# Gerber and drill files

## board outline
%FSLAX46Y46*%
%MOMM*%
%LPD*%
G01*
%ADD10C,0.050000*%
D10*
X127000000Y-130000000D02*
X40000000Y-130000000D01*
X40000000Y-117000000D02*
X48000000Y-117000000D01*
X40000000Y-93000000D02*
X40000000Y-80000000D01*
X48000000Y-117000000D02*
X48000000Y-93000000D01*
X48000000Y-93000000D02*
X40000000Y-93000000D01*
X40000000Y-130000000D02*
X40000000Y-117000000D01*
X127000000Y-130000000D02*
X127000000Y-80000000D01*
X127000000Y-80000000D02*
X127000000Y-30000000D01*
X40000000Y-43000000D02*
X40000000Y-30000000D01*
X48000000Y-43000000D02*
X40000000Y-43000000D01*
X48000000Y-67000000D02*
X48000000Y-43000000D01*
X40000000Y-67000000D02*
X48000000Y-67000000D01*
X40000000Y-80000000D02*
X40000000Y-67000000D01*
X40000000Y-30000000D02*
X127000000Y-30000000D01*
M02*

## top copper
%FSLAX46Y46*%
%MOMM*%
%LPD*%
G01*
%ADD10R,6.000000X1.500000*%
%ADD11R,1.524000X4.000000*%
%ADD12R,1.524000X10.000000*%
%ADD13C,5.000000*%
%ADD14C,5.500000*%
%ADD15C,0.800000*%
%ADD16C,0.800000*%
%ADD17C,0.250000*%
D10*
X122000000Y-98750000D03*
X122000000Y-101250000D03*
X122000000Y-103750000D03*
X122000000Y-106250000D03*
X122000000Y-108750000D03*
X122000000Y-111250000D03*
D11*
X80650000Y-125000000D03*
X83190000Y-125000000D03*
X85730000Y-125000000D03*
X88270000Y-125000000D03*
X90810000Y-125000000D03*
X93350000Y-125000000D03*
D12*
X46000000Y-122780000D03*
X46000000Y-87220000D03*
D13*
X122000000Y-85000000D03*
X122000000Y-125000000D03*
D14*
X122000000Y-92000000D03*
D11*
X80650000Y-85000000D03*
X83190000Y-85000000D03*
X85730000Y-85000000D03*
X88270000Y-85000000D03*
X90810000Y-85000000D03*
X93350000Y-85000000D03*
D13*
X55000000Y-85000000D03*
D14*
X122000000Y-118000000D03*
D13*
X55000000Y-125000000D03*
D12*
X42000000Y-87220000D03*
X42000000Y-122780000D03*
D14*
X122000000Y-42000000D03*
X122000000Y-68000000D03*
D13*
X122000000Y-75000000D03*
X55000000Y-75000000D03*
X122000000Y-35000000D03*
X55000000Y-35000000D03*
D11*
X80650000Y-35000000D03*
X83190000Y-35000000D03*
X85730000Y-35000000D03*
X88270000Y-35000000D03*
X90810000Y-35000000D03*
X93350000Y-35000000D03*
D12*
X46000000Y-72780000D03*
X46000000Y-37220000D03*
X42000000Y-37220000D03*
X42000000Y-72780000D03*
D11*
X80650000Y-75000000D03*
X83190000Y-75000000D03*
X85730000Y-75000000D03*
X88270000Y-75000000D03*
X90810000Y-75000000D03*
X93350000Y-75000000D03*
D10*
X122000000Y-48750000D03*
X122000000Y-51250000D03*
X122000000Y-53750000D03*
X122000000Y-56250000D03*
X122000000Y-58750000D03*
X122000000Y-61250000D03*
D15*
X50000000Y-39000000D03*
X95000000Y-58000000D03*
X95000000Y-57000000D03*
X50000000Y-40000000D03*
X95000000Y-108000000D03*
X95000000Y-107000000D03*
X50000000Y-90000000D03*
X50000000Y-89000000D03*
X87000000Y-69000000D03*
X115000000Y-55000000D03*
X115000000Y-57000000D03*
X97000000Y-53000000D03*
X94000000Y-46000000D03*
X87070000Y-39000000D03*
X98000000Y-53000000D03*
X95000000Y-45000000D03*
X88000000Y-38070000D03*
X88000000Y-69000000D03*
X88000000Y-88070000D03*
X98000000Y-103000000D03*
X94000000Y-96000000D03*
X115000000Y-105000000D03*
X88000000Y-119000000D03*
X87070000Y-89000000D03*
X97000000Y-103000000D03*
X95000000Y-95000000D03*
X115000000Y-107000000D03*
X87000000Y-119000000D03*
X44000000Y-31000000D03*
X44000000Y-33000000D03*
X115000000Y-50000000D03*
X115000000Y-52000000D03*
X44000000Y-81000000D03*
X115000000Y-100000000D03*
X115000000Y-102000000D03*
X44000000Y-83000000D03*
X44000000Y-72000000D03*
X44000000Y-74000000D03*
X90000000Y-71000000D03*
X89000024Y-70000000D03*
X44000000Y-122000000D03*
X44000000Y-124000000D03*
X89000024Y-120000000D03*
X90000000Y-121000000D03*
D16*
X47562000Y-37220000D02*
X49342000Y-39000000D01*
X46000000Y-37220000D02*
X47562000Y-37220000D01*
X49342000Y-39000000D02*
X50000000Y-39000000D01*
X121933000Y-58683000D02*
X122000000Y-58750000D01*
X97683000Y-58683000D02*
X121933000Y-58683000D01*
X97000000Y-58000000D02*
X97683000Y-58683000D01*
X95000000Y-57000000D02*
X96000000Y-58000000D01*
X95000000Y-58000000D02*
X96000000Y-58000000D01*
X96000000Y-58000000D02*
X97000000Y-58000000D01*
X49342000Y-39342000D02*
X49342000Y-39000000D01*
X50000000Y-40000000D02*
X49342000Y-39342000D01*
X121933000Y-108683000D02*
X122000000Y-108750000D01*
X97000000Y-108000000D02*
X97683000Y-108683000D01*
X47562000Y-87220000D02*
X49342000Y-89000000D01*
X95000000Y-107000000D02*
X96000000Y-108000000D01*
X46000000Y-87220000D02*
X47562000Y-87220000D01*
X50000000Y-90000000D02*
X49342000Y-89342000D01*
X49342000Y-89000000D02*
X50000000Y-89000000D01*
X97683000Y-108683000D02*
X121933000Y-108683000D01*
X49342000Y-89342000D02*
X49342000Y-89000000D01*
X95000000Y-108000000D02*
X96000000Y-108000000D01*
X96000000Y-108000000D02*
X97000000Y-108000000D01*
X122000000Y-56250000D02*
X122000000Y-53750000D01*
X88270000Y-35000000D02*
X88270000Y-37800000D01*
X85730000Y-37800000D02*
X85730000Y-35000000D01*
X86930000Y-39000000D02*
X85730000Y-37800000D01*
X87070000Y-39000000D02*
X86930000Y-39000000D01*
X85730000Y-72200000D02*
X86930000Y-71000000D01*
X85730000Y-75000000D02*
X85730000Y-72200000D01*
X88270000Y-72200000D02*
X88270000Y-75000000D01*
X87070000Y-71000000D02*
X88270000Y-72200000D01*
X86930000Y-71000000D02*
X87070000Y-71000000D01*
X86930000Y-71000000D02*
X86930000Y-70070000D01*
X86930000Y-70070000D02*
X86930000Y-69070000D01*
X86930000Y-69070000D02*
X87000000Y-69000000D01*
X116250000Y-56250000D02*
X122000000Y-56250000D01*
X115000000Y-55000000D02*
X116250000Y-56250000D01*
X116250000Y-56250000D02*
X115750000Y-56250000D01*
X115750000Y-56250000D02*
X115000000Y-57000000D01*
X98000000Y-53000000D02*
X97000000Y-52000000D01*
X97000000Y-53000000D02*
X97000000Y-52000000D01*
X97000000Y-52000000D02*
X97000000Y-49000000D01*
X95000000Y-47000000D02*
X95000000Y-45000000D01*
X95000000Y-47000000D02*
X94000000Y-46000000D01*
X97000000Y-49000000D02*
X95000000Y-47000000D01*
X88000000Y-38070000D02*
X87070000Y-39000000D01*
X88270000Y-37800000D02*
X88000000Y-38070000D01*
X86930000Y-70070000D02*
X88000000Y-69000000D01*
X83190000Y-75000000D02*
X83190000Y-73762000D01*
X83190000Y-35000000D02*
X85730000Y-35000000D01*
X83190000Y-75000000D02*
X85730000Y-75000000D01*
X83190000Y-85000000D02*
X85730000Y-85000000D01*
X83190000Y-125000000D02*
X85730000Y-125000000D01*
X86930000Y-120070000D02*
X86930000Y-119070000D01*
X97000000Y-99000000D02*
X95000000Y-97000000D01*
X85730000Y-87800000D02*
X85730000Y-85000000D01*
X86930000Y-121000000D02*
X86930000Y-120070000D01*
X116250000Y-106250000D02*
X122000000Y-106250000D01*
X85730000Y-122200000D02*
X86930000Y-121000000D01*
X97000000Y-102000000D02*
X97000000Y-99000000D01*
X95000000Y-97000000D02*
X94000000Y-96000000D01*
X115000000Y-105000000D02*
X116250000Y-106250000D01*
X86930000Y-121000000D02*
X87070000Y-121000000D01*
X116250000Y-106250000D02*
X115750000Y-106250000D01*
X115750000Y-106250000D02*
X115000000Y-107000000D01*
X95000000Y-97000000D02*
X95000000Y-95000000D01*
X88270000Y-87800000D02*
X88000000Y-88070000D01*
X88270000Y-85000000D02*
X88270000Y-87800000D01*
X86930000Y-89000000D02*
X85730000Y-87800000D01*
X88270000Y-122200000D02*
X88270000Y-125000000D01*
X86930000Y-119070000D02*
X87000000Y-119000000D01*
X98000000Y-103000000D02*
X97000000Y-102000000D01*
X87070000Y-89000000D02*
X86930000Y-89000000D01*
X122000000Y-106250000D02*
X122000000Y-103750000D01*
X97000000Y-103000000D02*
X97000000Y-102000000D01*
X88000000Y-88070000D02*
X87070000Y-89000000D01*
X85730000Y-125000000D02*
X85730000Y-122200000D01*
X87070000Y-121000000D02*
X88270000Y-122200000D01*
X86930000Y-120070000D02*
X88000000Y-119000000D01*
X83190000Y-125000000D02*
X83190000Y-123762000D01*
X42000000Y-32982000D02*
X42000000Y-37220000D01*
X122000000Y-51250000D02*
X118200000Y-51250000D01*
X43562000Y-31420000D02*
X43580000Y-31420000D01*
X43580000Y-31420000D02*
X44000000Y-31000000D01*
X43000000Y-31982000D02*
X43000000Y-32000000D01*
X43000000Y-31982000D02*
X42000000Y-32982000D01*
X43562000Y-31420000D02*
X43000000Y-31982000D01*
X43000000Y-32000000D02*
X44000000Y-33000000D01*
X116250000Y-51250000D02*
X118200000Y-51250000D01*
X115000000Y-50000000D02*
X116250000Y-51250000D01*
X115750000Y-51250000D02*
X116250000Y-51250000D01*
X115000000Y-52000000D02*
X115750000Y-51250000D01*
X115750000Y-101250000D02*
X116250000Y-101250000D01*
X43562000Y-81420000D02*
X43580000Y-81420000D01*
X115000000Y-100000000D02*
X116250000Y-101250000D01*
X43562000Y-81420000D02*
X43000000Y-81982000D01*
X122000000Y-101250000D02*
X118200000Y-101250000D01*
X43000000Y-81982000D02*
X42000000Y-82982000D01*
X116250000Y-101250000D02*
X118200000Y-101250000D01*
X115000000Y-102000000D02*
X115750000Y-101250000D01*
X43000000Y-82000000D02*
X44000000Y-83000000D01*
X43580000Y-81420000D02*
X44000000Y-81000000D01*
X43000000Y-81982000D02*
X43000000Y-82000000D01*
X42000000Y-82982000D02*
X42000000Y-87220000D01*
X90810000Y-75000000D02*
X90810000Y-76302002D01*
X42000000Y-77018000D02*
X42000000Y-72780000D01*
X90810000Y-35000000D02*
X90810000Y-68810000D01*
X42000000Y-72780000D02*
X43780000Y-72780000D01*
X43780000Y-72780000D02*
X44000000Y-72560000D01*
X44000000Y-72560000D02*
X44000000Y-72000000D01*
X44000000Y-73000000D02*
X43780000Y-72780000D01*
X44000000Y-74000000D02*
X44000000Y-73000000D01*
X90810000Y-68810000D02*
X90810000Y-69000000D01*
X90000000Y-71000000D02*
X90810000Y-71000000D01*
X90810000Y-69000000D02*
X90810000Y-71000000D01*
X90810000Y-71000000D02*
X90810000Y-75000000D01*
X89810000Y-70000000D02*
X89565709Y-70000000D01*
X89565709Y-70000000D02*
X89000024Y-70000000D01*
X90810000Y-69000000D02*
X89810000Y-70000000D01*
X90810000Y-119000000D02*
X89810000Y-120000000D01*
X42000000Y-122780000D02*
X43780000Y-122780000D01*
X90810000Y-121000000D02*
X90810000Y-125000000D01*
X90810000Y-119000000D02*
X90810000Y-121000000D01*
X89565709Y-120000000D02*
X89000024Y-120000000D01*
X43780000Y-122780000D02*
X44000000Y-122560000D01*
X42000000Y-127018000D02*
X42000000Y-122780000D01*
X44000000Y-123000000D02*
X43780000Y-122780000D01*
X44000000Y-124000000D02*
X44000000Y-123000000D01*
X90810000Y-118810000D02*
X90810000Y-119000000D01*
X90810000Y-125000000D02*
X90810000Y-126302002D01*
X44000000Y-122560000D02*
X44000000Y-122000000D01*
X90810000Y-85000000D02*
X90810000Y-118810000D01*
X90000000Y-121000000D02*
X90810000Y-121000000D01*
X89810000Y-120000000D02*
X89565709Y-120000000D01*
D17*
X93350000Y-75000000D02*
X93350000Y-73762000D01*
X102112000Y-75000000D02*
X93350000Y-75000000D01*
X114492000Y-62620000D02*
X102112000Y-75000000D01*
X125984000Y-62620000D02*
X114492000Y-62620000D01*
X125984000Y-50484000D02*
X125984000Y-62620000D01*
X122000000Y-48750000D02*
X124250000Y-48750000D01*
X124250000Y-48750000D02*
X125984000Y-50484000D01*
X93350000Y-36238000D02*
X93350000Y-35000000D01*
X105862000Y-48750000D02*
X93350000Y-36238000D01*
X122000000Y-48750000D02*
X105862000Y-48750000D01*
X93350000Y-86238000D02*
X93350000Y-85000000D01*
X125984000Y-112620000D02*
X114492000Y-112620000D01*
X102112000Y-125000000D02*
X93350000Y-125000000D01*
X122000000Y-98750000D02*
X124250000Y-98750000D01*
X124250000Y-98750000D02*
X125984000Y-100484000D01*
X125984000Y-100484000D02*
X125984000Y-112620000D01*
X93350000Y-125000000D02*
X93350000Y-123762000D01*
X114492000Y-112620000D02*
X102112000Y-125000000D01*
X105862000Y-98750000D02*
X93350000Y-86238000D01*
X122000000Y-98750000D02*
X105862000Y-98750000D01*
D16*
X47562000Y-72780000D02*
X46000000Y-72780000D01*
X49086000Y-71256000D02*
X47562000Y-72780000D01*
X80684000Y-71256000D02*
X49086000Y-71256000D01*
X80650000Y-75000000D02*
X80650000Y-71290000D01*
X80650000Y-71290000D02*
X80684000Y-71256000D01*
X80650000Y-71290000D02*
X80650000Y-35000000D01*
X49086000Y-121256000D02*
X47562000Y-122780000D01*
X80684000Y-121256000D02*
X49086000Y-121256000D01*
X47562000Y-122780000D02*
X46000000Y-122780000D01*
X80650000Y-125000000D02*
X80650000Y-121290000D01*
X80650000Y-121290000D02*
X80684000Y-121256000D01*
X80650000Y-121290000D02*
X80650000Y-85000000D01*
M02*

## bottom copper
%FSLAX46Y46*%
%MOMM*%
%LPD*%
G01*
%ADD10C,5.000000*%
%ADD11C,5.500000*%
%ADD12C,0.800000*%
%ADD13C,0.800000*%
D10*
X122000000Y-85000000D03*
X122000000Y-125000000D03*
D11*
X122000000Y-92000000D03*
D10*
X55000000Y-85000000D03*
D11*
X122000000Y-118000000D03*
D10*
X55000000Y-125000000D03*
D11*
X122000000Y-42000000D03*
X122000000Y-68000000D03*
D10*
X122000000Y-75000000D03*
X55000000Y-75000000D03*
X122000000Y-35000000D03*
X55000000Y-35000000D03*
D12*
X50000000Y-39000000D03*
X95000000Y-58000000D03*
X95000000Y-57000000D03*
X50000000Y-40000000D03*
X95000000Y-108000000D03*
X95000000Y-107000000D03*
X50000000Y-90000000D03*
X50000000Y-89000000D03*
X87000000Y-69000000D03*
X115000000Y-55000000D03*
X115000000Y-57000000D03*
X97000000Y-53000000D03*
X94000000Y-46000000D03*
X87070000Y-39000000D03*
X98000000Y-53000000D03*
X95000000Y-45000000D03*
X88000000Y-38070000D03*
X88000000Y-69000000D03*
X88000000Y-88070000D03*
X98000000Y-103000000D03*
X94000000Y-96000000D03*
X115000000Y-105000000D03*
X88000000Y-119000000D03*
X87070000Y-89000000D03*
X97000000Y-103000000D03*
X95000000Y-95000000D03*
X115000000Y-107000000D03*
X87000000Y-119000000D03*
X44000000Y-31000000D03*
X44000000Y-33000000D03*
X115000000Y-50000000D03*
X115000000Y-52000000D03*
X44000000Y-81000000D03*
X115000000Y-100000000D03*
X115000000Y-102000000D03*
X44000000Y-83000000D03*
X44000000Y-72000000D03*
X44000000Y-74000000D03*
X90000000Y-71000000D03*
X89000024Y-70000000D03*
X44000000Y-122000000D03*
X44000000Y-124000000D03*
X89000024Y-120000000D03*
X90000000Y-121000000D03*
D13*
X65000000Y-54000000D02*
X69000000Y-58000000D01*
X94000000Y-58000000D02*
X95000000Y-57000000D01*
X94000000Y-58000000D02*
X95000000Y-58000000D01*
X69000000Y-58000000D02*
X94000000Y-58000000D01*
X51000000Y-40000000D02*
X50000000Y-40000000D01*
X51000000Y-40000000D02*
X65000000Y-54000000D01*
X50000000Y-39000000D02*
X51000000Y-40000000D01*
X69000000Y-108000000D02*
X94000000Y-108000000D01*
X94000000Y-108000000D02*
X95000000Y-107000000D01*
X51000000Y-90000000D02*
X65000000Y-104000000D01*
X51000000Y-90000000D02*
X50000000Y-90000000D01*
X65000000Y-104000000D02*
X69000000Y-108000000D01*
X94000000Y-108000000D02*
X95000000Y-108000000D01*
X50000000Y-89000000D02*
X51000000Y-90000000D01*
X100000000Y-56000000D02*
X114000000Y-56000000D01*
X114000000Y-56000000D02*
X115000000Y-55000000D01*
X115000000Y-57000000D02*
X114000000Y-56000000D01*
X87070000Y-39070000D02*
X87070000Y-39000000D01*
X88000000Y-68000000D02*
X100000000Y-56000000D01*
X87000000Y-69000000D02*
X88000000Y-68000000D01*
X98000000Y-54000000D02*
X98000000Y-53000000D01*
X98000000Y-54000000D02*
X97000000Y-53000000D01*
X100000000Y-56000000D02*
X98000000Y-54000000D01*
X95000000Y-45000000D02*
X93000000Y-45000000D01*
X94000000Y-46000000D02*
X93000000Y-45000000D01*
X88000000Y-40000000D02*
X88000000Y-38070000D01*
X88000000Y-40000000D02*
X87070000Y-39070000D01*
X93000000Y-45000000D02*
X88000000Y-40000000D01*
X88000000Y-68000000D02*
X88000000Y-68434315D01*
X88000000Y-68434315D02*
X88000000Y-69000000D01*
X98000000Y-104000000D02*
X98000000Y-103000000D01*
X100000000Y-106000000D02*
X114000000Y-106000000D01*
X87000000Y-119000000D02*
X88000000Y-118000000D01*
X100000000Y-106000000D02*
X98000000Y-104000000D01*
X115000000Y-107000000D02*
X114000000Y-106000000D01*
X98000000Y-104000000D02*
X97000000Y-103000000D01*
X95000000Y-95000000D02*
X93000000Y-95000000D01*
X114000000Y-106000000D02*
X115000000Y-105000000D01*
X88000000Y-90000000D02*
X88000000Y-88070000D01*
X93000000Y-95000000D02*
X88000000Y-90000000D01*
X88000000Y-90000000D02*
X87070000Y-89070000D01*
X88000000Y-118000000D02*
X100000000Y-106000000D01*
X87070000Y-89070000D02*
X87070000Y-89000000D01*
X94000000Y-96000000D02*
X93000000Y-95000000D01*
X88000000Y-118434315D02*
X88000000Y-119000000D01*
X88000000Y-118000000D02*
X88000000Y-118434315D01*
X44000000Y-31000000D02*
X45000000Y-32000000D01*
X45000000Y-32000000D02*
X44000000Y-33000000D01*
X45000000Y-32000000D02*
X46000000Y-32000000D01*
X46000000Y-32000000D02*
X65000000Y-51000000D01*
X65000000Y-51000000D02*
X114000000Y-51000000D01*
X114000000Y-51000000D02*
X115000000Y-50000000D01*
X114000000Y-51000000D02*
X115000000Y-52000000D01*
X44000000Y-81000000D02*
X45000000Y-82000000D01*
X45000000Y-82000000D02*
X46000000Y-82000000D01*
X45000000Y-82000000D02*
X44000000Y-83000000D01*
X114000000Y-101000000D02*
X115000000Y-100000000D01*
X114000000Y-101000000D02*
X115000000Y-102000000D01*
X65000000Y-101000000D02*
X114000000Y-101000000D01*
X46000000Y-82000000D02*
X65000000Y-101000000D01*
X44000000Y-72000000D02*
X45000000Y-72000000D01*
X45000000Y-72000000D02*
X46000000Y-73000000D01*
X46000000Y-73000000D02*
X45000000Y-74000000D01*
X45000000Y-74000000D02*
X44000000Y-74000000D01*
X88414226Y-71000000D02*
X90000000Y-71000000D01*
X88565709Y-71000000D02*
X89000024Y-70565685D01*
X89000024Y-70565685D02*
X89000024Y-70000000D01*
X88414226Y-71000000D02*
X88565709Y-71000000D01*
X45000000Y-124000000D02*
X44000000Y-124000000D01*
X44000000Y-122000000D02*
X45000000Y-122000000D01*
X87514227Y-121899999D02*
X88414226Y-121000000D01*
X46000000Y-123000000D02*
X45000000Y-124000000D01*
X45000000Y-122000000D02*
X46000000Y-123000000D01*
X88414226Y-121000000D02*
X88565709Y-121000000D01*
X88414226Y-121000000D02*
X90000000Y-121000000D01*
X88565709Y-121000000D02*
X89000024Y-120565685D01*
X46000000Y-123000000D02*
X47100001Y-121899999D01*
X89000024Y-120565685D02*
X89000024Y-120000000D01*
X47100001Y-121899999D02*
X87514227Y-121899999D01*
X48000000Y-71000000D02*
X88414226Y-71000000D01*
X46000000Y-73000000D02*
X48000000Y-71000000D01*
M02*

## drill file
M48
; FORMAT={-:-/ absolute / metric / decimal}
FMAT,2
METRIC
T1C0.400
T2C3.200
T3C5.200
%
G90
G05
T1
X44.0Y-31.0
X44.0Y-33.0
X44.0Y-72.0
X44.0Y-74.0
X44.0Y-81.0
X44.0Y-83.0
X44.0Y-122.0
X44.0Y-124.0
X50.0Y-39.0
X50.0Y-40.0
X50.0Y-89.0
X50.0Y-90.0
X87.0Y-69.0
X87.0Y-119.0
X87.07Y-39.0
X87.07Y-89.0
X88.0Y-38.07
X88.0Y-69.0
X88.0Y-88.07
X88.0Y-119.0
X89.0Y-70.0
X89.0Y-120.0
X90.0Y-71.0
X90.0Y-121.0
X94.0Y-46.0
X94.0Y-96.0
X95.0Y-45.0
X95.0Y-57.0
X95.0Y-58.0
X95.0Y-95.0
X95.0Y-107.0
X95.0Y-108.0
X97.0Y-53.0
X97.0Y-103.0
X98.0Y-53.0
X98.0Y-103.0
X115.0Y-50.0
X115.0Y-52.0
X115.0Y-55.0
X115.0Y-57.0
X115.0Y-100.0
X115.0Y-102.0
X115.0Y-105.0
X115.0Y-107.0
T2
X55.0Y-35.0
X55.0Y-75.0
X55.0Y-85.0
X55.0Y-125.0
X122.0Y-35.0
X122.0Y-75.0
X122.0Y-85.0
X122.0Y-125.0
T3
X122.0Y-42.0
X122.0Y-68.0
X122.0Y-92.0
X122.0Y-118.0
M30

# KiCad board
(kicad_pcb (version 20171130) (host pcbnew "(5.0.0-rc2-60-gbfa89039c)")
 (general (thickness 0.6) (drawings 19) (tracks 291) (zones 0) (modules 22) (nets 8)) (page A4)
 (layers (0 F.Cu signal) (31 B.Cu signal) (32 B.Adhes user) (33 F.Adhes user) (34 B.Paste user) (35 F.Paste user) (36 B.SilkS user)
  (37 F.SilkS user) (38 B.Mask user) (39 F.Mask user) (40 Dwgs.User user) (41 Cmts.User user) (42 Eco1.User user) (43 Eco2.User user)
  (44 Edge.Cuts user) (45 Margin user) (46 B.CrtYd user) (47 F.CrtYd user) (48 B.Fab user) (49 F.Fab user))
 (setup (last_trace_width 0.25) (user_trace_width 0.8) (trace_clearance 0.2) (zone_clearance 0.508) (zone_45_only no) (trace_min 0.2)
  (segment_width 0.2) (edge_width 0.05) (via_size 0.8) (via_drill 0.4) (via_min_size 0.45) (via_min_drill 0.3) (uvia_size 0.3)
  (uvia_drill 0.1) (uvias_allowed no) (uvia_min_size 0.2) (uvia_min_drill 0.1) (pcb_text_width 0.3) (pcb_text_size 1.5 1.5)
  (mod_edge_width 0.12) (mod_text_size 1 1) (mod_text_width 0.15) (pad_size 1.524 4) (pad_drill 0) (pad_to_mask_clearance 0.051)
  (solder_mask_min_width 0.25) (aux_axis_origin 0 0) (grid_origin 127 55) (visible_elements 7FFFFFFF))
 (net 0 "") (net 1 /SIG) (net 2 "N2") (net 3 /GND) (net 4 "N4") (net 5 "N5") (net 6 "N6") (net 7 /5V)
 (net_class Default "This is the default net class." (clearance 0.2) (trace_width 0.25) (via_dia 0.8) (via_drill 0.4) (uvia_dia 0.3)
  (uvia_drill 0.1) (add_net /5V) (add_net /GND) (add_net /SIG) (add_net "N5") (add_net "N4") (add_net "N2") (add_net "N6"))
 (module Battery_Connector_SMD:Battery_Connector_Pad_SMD (layer F.Cu) (at 122 105 90)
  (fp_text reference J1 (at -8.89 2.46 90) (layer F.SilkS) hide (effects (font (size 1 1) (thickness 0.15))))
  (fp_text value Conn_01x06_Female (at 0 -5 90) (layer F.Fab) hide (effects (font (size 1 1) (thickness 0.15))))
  (pad 6 smd rect (at 6.25 0 90) (size 1.5 6) (layers F.Cu F.Mask) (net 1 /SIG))
  (pad 5 smd rect (at 3.75 0 90) (size 1.5 6) (layers F.Cu F.Mask) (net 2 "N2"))
  (pad 4 smd rect (at 1.25 0 90) (size 1.5 6) (layers F.Cu F.Mask) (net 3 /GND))
  (pad 3 smd rect (at -1.25 0 90) (size 1.5 6) (layers F.Cu F.Mask) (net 3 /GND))
  (pad 2 smd rect (at -3.75 0 90) (size 1.5 6) (layers F.Cu F.Mask) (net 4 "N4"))
  (pad 1 smd rect (at -6.25 0 90) (size 1.5 6) (layers F.Cu F.Mask) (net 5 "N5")))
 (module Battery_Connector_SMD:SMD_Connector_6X (layer F.Cu) (at 87 125 180)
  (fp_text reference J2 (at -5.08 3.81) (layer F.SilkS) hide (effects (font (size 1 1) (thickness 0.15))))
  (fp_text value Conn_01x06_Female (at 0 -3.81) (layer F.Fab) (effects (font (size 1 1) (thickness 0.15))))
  (pad 6 smd rect (at 6.35 0 180) (size 1.524 4) (layers F.Cu F.Paste F.Mask) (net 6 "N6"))
  (pad 5 smd rect (at 3.81 0 180) (size 1.524 4) (layers F.Cu F.Paste F.Mask) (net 3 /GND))
  (pad 4 smd rect (at 1.27 0 180) (size 1.524 4) (layers F.Cu F.Paste F.Mask) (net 3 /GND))
  (pad 3 smd rect (at -1.27 0 180) (size 1.524 4) (layers F.Cu F.Paste F.Mask) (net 3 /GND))
  (pad 2 smd rect (at -3.81 0 180) (size 1.524 4) (layers F.Cu F.Paste F.Mask) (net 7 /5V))
  (pad 1 smd rect (at -6.35 0 180) (size 1.524 4) (layers F.Cu F.Paste F.Mask) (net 1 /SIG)))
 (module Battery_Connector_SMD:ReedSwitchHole (layer F.Cu) (at 46 105)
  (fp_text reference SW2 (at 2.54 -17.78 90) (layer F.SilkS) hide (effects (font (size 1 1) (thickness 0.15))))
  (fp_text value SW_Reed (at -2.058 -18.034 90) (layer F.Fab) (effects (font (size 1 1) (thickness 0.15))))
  (pad 2 smd rect (at 0 17.78) (size 1.524 10) (layers F.Cu F.Mask) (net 6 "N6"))
  (pad 1 smd rect (at 0 -17.78) (size 1.524 10) (layers F.Cu F.Mask) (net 4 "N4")))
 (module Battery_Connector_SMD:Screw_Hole (layer F.Cu) (at 122 85)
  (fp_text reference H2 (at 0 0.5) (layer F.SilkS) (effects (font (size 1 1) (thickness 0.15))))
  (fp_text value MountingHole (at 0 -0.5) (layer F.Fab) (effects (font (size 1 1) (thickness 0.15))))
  (pad 1 thru_hole circle (at 0 0) (size 5 5) (drill 3.2) (layers *.Cu *.Mask)))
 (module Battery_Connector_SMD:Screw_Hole (layer F.Cu) (at 122 125)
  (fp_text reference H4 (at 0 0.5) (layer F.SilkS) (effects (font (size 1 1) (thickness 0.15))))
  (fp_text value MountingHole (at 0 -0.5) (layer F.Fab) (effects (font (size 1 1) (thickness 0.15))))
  (pad 1 thru_hole circle (at 0 0) (size 5 5) (drill 3.2) (layers *.Cu *.Mask)))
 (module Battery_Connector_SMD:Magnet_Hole (layer F.Cu) (at 122 92)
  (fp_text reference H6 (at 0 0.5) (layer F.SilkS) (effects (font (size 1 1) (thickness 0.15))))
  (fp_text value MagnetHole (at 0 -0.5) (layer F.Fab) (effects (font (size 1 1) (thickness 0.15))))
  (pad 1 thru_hole circle (at 0 0) (size 5.5 5.5) (drill 5.2) (layers *.Cu *.Mask)))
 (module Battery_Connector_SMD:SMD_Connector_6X (layer F.Cu) (at 87 85 180)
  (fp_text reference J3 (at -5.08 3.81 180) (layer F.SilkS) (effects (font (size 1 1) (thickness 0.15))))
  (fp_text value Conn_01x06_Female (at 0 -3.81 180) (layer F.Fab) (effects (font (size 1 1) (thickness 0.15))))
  (pad 6 smd rect (at 6.35 0 180) (size 1.524 4) (layers F.Cu F.Paste F.Mask) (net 6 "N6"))
  (pad 5 smd rect (at 3.81 0 180) (size 1.524 4) (layers F.Cu F.Paste F.Mask) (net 3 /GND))
  (pad 4 smd rect (at 1.27 0 180) (size 1.524 4) (layers F.Cu F.Paste F.Mask) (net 3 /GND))
  (pad 3 smd rect (at -1.27 0 180) (size 1.524 4) (layers F.Cu F.Paste F.Mask) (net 3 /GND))
  (pad 2 smd rect (at -3.81 0 180) (size 1.524 4) (layers F.Cu F.Paste F.Mask) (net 7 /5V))
  (pad 1 smd rect (at -6.35 0 180) (size 1.524 4) (layers F.Cu F.Paste F.Mask) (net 1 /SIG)))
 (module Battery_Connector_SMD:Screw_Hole (layer F.Cu) (at 55 85)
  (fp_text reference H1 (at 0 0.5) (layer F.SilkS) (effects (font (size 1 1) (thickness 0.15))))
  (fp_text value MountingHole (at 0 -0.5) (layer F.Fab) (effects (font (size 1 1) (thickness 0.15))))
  (pad 1 thru_hole circle (at 0 0) (size 5 5) (drill 3.2) (layers *.Cu *.Mask)))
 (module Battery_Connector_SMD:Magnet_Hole (layer F.Cu) (at 122 118)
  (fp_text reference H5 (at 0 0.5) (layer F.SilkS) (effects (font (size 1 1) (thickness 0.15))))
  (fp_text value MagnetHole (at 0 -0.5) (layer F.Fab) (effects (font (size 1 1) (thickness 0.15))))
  (pad 1 thru_hole circle (at 0 0) (size 5.5 5.5) (drill 5.2) (layers *.Cu *.Mask)))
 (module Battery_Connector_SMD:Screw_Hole (layer F.Cu) (at 55 125)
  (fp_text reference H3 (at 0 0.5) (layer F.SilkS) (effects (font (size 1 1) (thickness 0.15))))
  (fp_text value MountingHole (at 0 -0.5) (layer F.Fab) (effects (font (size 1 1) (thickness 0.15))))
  (pad 1 thru_hole circle (at 0 0) (size 5 5) (drill 3.2) (layers *.Cu *.Mask)))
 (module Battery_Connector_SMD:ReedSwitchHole (layer F.Cu) (at 42 105 180)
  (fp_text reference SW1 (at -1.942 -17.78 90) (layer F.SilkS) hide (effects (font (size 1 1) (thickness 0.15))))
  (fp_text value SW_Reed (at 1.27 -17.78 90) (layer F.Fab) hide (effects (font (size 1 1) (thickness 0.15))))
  (pad 2 smd rect (at 0 17.78 180) (size 1.524 10) (layers F.Cu F.Mask) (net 2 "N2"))
  (pad 1 smd rect (at 0 -17.78 180) (size 1.524 10) (layers F.Cu F.Mask) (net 7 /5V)))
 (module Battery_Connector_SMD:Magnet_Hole (layer F.Cu) (at 122 42)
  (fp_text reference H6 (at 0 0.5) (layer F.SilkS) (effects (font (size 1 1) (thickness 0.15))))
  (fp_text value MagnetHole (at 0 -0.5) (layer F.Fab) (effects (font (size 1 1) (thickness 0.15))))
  (pad 1 thru_hole circle (at 0 0) (size 5.5 5.5) (drill 5.2) (layers *.Cu *.Mask)))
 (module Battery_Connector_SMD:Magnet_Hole (layer F.Cu) (at 122 68)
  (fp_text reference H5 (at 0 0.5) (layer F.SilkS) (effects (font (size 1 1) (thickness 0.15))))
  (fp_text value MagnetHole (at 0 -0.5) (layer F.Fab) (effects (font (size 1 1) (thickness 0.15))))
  (pad 1 thru_hole circle (at 0 0) (size 5.5 5.5) (drill 5.2) (layers *.Cu *.Mask)))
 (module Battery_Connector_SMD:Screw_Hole (layer F.Cu) (at 122 75)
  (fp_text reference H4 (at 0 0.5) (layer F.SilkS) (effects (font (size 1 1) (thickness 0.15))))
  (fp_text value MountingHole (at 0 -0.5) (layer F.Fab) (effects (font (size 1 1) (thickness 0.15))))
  (pad 1 thru_hole circle (at 0 0) (size 5 5) (drill 3.2) (layers *.Cu *.Mask)))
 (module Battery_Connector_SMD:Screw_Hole (layer F.Cu) (at 55 75)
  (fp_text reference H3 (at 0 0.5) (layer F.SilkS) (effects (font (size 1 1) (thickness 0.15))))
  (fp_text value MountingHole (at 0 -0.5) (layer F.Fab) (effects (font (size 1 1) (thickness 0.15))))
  (pad 1 thru_hole circle (at 0 0) (size 5 5) (drill 3.2) (layers *.Cu *.Mask)))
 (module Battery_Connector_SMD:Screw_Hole (layer F.Cu) (at 122 35)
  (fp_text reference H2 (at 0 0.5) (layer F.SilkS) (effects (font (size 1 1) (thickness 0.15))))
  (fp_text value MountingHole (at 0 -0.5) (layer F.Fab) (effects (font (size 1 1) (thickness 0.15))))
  (pad 1 thru_hole circle (at 0 0) (size 5 5) (drill 3.2) (layers *.Cu *.Mask)))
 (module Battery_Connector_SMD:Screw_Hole (layer F.Cu) (at 55 35)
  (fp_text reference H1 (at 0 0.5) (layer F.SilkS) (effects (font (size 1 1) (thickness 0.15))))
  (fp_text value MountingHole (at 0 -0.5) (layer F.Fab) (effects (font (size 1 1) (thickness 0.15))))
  (pad 1 thru_hole circle (at 0 0) (size 5 5) (drill 3.2) (layers *.Cu *.Mask)))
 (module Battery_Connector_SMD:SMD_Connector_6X (layer F.Cu) (at 87 35 180)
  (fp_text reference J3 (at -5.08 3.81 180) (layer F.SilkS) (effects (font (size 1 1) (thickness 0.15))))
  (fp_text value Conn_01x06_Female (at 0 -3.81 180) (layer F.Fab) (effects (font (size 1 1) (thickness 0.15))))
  (pad 6 smd rect (at 6.35 0 180) (size 1.524 4) (layers F.Cu F.Paste F.Mask) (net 6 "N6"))
  (pad 5 smd rect (at 3.81 0 180) (size 1.524 4) (layers F.Cu F.Paste F.Mask) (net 3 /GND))
  (pad 4 smd rect (at 1.27 0 180) (size 1.524 4) (layers F.Cu F.Paste F.Mask) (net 3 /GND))
  (pad 3 smd rect (at -1.27 0 180) (size 1.524 4) (layers F.Cu F.Paste F.Mask) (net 3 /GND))
  (pad 2 smd rect (at -3.81 0 180) (size 1.524 4) (layers F.Cu F.Paste F.Mask) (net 7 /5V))
  (pad 1 smd rect (at -6.35 0 180) (size 1.524 4) (layers F.Cu F.Paste F.Mask) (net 1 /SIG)))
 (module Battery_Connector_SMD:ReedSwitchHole (layer F.Cu) (at 46 55)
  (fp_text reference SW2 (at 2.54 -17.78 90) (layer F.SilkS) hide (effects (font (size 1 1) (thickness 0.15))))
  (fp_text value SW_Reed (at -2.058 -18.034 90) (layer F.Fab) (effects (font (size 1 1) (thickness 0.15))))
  (pad 2 smd rect (at 0 17.78) (size 1.524 10) (layers F.Cu F.Mask) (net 6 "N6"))
  (pad 1 smd rect (at 0 -17.78) (size 1.524 10) (layers F.Cu F.Mask) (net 4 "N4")))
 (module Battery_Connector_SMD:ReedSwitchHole (layer F.Cu) (at 42 55 180)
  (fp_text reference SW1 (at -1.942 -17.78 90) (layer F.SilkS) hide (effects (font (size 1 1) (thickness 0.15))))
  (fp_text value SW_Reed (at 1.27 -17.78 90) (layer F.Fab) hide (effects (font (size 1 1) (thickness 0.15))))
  (pad 2 smd rect (at 0 17.78 180) (size 1.524 10) (layers F.Cu F.Mask) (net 2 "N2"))
  (pad 1 smd rect (at 0 -17.78 180) (size 1.524 10) (layers F.Cu F.Mask) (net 7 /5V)))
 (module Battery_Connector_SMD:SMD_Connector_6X (layer F.Cu) (at 87 75 180)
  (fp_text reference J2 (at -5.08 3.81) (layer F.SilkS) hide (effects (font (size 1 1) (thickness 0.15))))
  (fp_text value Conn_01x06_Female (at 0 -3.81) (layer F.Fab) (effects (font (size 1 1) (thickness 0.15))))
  (pad 6 smd rect (at 6.35 0 180) (size 1.524 4) (layers F.Cu F.Paste F.Mask) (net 6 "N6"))
  (pad 5 smd rect (at 3.81 0 180) (size 1.524 4) (layers F.Cu F.Paste F.Mask) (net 3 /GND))
  (pad 4 smd rect (at 1.27 0 180) (size 1.524 4) (layers F.Cu F.Paste F.Mask) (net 3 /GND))
  (pad 3 smd rect (at -1.27 0 180) (size 1.524 4) (layers F.Cu F.Paste F.Mask) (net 3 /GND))
  (pad 2 smd rect (at -3.81 0 180) (size 1.524 4) (layers F.Cu F.Paste F.Mask) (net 7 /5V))
  (pad 1 smd rect (at -6.35 0 180) (size 1.524 4) (layers F.Cu F.Paste F.Mask) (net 1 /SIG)))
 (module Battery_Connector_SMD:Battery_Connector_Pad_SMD (layer F.Cu) (at 122 55 90)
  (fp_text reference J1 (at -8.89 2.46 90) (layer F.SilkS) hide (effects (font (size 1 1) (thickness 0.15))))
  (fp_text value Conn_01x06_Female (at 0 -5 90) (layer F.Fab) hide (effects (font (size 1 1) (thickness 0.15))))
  (pad 6 smd rect (at 6.25 0 90) (size 1.5 6) (layers F.Cu F.Mask) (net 1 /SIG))
  (pad 5 smd rect (at 3.75 0 90) (size 1.5 6) (layers F.Cu F.Mask) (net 2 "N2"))
  (pad 4 smd rect (at 1.25 0 90) (size 1.5 6) (layers F.Cu F.Mask) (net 3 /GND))
  (pad 3 smd rect (at -1.25 0 90) (size 1.5 6) (layers F.Cu F.Mask) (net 3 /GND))
  (pad 2 smd rect (at -3.75 0 90) (size 1.5 6) (layers F.Cu F.Mask) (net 4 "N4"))
  (pad 1 smd rect (at -6.25 0 90) (size 1.5 6) (layers F.Cu F.Mask) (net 5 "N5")))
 (gr_line (start 127 130) (end 40 130) (layer Edge.Cuts) (width 0.05))
 (gr_line (start 40 117) (end 48 117) (layer Edge.Cuts) (width 0.05))
 (gr_line (start 40 93) (end 40 80) (layer Edge.Cuts) (width 0.05))
 (gr_line (start 48 117) (end 48 93) (layer Edge.Cuts) (width 0.05))
 (gr_line (start 48 93) (end 40 93) (layer Edge.Cuts) (width 0.05))
 (gr_line (start 40 130) (end 40 117) (layer Edge.Cuts) (width 0.05))
 (gr_line (start 127 130) (end 127 80) (layer Edge.Cuts) (width 0.05))
 (gr_line (start 127 80) (end 127 30) (layer Edge.Cuts) (width 0.05))
 (gr_line (start 40 43) (end 40 30) (layer Edge.Cuts) (width 0.05))
 (gr_line (start 48 43) (end 40 43) (layer Edge.Cuts) (width 0.05))
 (gr_line (start 48 67) (end 48 43) (layer Edge.Cuts) (width 0.05))
 (gr_line (start 40 67) (end 48 67) (layer Edge.Cuts) (width 0.05))
 (gr_line (start 40 80) (end 40 67) (layer Edge.Cuts) (width 0.05))
 (gr_line (start 40 30) (end 127 30) (layer Edge.Cuts) (width 0.05))
 (segment (start 47.562 37.22) (end 49.342 39) (width 0.8) (layer F.Cu) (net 4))
 (segment (start 46 37.22) (end 47.562 37.22) (width 0.8) (layer F.Cu) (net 4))
 (via (at 50 39) (size 0.8) (drill 0.4) (layers F.Cu B.Cu) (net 4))
 (segment (start 49.342 39) (end 50 39) (width 0.8) (layer F.Cu) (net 4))
 (segment (start 65 54) (end 69 58) (width 0.8) (layer B.Cu) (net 4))
 (via (at 95 58) (size 0.8) (drill 0.4) (layers F.Cu B.Cu) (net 4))
 (segment (start 121.933 58.683) (end 122 58.75) (width 0.8) (layer F.Cu) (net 4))
 (segment (start 97.683 58.683) (end 121.933 58.683) (width 0.8) (layer F.Cu) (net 4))
 (segment (start 97 58) (end 97.683 58.683) (width 0.8) (layer F.Cu) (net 4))
 (via (at 95 57) (size 0.8) (drill 0.4) (layers F.Cu B.Cu) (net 4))
 (segment (start 94 58) (end 95 57) (width 0.8) (layer B.Cu) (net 4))
 (segment (start 94 58) (end 95 58) (width 0.8) (layer B.Cu) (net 4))
 (segment (start 69 58) (end 94 58) (width 0.8) (layer B.Cu) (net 4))
 (segment (start 95 57) (end 96 58) (width 0.8) (layer F.Cu) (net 4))
 (segment (start 95 58) (end 96 58) (width 0.8) (layer F.Cu) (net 4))
 (segment (start 96 58) (end 97 58) (width 0.8) (layer F.Cu) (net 4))
 (via (at 50 40) (size 0.8) (drill 0.4) (layers F.Cu B.Cu) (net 4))
 (segment (start 51 40) (end 50 40) (width 0.8) (layer B.Cu) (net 4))
 (segment (start 51 40) (end 65 54) (width 0.8) (layer B.Cu) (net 4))
 (segment (start 50 39) (end 51 40) (width 0.8) (layer B.Cu) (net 4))
 (segment (start 49.342 39.342) (end 49.342 39) (width 0.8) (layer F.Cu) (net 4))
 (segment (start 50 40) (end 49.342 39.342) (width 0.8) (layer F.Cu) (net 4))
 (segment (start 121.933 108.683) (end 122 108.75) (width 0.8) (layer F.Cu) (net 4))
 (segment (start 69 108) (end 94 108) (width 0.8) (layer B.Cu) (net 4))
 (segment (start 94 108) (end 95 107) (width 0.8) (layer B.Cu) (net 4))
 (segment (start 51 90) (end 65 104) (width 0.8) (layer B.Cu) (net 4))
 (segment (start 97 108) (end 97.683 108.683) (width 0.8) (layer F.Cu) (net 4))
 (segment (start 47.562 87.22) (end 49.342 89) (width 0.8) (layer F.Cu) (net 4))
 (segment (start 95 107) (end 96 108) (width 0.8) (layer F.Cu) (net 4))
 (segment (start 51 90) (end 50 90) (width 0.8) (layer B.Cu) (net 4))
 (segment (start 46 87.22) (end 47.562 87.22) (width 0.8) (layer F.Cu) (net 4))
 (segment (start 50 90) (end 49.342 89.342) (width 0.8) (layer F.Cu) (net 4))
 (segment (start 49.342 89) (end 50 89) (width 0.8) (layer F.Cu) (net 4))
 (segment (start 65 104) (end 69 108) (width 0.8) (layer B.Cu) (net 4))
 (segment (start 94 108) (end 95 108) (width 0.8) (layer B.Cu) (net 4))
 (segment (start 97.683 108.683) (end 121.933 108.683) (width 0.8) (layer F.Cu) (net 4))
 (segment (start 49.342 89.342) (end 49.342 89) (width 0.8) (layer F.Cu) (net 4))
 (segment (start 95 108) (end 96 108) (width 0.8) (layer F.Cu) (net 4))
 (segment (start 96 108) (end 97 108) (width 0.8) (layer F.Cu) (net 4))
 (segment (start 50 89) (end 51 90) (width 0.8) (layer B.Cu) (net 4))
 (via (at 95 108) (size 0.8) (drill 0.4) (layers F.Cu B.Cu) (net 4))
 (via (at 95 107) (size 0.8) (drill 0.4) (layers F.Cu B.Cu) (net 4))
 (via (at 50 90) (size 0.8) (drill 0.4) (layers F.Cu B.Cu) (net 4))
 (via (at 50 89) (size 0.8) (drill 0.4) (layers F.Cu B.Cu) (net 4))
 (segment (start 122 56.25) (end 122 53.75) (width 0.8) (layer F.Cu) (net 3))
 (segment (start 88.27 35) (end 88.27 37.8) (width 0.8) (layer F.Cu) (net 3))
 (segment (start 85.73 37.8) (end 85.73 35) (width 0.8) (layer F.Cu) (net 3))
 (segment (start 86.93 39) (end 85.73 37.8) (width 0.8) (layer F.Cu) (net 3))
 (segment (start 87.07 39) (end 86.93 39) (width 0.8) (layer F.Cu) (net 3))
 (segment (start 85.73 72.2) (end 86.93 71) (width 0.8) (layer F.Cu) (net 3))
 (segment (start 85.73 75) (end 85.73 72.2) (width 0.8) (layer F.Cu) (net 3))
 (segment (start 88.27 72.2) (end 88.27 75) (width 0.8) (layer F.Cu) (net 3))
 (segment (start 87.07 71) (end 88.27 72.2) (width 0.8) (layer F.Cu) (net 3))
 (segment (start 86.93 71) (end 87.07 71) (width 0.8) (layer F.Cu) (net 3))
 (segment (start 86.93 71) (end 86.93 70.07) (width 0.8) (layer F.Cu) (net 3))
 (via (at 87 69) (size 0.8) (drill 0.4) (layers F.Cu B.Cu) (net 3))
 (segment (start 86.93 70.07) (end 86.93 69.07) (width 0.8) (layer F.Cu) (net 3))
 (segment (start 86.93 69.07) (end 87 69) (width 0.8) (layer F.Cu) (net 3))
 (segment (start 100 56) (end 114 56) (width 0.8) (layer B.Cu) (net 3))
 (via (at 115 55) (size 0.8) (drill 0.4) (layers F.Cu B.Cu) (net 3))
 (segment (start 114 56) (end 115 55) (width 0.8) (layer B.Cu) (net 3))
 (segment (start 116.25 56.25) (end 122 56.25) (width 0.8) (layer F.Cu) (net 3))
 (segment (start 115 55) (end 116.25 56.25) (width 0.8) (layer F.Cu) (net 3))
 (via (at 115 57) (size 0.8) (drill 0.4) (layers F.Cu B.Cu) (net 3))
 (segment (start 116.25 56.25) (end 115.75 56.25) (width 0.8) (layer F.Cu) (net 3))
 (segment (start 115.75 56.25) (end 115 57) (width 0.8) (layer F.Cu) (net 3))
 (segment (start 115 57) (end 114 56) (width 0.8) (layer B.Cu) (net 3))
 (via (at 97 53) (size 0.8) (drill 0.4) (layers F.Cu B.Cu) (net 3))
 (via (at 94 46) (size 0.8) (drill 0.4) (layers F.Cu B.Cu) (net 3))
 (via (at 87.07 39) (size 0.8) (drill 0.4) (layers F.Cu B.Cu) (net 3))
 (segment (start 87.07 39.07) (end 87.07 39) (width 0.8) (layer B.Cu) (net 3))
 (segment (start 88 68) (end 100 56) (width 0.8) (layer B.Cu) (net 3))
 (segment (start 87 69) (end 88 68) (width 0.8) (layer B.Cu) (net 3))
 (via (at 98 53) (size 0.8) (drill 0.4) (layers F.Cu B.Cu) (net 3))
 (segment (start 98 54) (end 98 53) (width 0.8) (layer B.Cu) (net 3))
 (segment (start 98 54) (end 97 53) (width 0.8) (layer B.Cu) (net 3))
 (segment (start 100 56) (end 98 54) (width 0.8) (layer B.Cu) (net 3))
 (segment (start 98 53) (end 97 52) (width 0.8) (layer F.Cu) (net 3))
 (segment (start 97 53) (end 97 52) (width 0.8) (layer F.Cu) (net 3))
 (segment (start 97 52) (end 97 49) (width 0.8) (layer F.Cu) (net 3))
 (via (at 95 45) (size 0.8) (drill 0.4) (layers F.Cu B.Cu) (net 3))
 (segment (start 95 47) (end 95 45) (width 0.8) (layer F.Cu) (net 3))
 (segment (start 95 47) (end 94 46) (width 0.8) (layer F.Cu) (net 3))
 (segment (start 97 49) (end 95 47) (width 0.8) (layer F.Cu) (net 3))
 (segment (start 95 45) (end 93 45) (width 0.8) (layer B.Cu) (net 3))
 (segment (start 94 46) (end 93 45) (width 0.8) (layer B.Cu) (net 3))
 (via (at 88 38.07) (size 0.8) (drill 0.4) (layers F.Cu B.Cu) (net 3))
 (segment (start 88 40) (end 88 38.07) (width 0.8) (layer B.Cu) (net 3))
 (segment (start 88 38.07) (end 87.07 39) (width 0.8) (layer F.Cu) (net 3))
 (segment (start 88.27 37.8) (end 88 38.07) (width 0.8) (layer F.Cu) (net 3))
 (segment (start 88 40) (end 87.07 39.07) (width 0.8) (layer B.Cu) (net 3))
 (segment (start 93 45) (end 88 40) (width 0.8) (layer B.Cu) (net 3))
 (segment (start 88 68) (end 88 68.434315) (width 0.8) (layer B.Cu) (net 3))
 (via (at 88 69) (size 0.8) (drill 0.4) (layers F.Cu B.Cu) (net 3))
 (segment (start 86.93 70.07) (end 88 69) (width 0.8) (layer F.Cu) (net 3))
 (segment (start 88 68.434315) (end 88 69) (width 0.8) (layer B.Cu) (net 3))
 (segment (start 83.19 75) (end 83.19 73.762) (width 0.8) (layer F.Cu) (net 3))
 (segment (start 83.19 35) (end 85.73 35) (width 0.8) (layer F.Cu) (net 3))
 (segment (start 83.19 75) (end 85.73 75) (width 0.8) (layer F.Cu) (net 3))
 (segment (start 83.19 85) (end 85.73 85) (width 0.8) (layer F.Cu) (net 3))
 (segment (start 83.19 125) (end 85.73 125) (width 0.8) (layer F.Cu) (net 3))
 (segment (start 86.93 120.07) (end 86.93 119.07) (width 0.8) (layer F.Cu) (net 3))
 (segment (start 98 104) (end 98 103) (width 0.8) (layer B.Cu) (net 3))
 (segment (start 97 99) (end 95 97) (width 0.8) (layer F.Cu) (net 3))
 (segment (start 85.73 87.8) (end 85.73 85) (width 0.8) (layer F.Cu) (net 3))
 (segment (start 86.93 121) (end 86.93 120.07) (width 0.8) (layer F.Cu) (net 3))
 (segment (start 116.25 106.25) (end 122 106.25) (width 0.8) (layer F.Cu) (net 3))
 (segment (start 85.73 122.2) (end 86.93 121) (width 0.8) (layer F.Cu) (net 3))
 (segment (start 100 106) (end 114 106) (width 0.8) (layer B.Cu) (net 3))
 (segment (start 87 119) (end 88 118) (width 0.8) (layer B.Cu) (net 3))
 (segment (start 97 102) (end 97 99) (width 0.8) (layer F.Cu) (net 3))
 (segment (start 100 106) (end 98 104) (width 0.8) (layer B.Cu) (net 3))
 (segment (start 115 107) (end 114 106) (width 0.8) (layer B.Cu) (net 3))
 (segment (start 98 104) (end 97 103) (width 0.8) (layer B.Cu) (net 3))
 (segment (start 95 95) (end 93 95) (width 0.8) (layer B.Cu) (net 3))
 (segment (start 95 97) (end 94 96) (width 0.8) (layer F.Cu) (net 3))
 (segment (start 115 105) (end 116.25 106.25) (width 0.8) (layer F.Cu) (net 3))
 (segment (start 86.93 121) (end 87.07 121) (width 0.8) (layer F.Cu) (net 3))
 (segment (start 116.25 106.25) (end 115.75 106.25) (width 0.8) (layer F.Cu) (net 3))
 (segment (start 114 106) (end 115 105) (width 0.8) (layer B.Cu) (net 3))
 (segment (start 115.75 106.25) (end 115 107) (width 0.8) (layer F.Cu) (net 3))
 (segment (start 95 97) (end 95 95) (width 0.8) (layer F.Cu) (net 3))
 (segment (start 88 90) (end 88 88.07) (width 0.8) (layer B.Cu) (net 3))
 (segment (start 88.27 87.8) (end 88 88.07) (width 0.8) (layer F.Cu) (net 3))
 (segment (start 93 95) (end 88 90) (width 0.8) (layer B.Cu) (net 3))
 (segment (start 88.27 85) (end 88.27 87.8) (width 0.8) (layer F.Cu) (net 3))
 (segment (start 86.93 89) (end 85.73 87.8) (width 0.8) (layer F.Cu) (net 3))
 (segment (start 88.27 122.2) (end 88.27 125) (width 0.8) (layer F.Cu) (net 3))
 (segment (start 86.93 119.07) (end 87 119) (width 0.8) (layer F.Cu) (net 3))
 (segment (start 88 90) (end 87.07 89.07) (width 0.8) (layer B.Cu) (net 3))
 (segment (start 88 118) (end 100 106) (width 0.8) (layer B.Cu) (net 3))
 (segment (start 98 103) (end 97 102) (width 0.8) (layer F.Cu) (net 3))
 (segment (start 87.07 89) (end 86.93 89) (width 0.8) (layer F.Cu) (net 3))
 (segment (start 87.07 89.07) (end 87.07 89) (width 0.8) (layer B.Cu) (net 3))
 (segment (start 122 106.25) (end 122 103.75) (width 0.8) (layer F.Cu) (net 3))
 (segment (start 97 103) (end 97 102) (width 0.8) (layer F.Cu) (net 3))
 (segment (start 94 96) (end 93 95) (width 0.8) (layer B.Cu) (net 3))
 (segment (start 88 88.07) (end 87.07 89) (width 0.8) (layer F.Cu) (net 3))
 (segment (start 85.73 125) (end 85.73 122.2) (width 0.8) (layer F.Cu) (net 3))
 (segment (start 87.07 121) (end 88.27 122.2) (width 0.8) (layer F.Cu) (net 3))
 (segment (start 88 118.434315) (end 88 119) (width 0.8) (layer B.Cu) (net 3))
 (segment (start 86.93 120.07) (end 88 119) (width 0.8) (layer F.Cu) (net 3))
 (segment (start 88 118) (end 88 118.434315) (width 0.8) (layer B.Cu) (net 3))
 (segment (start 83.19 125) (end 83.19 123.762) (width 0.8) (layer F.Cu) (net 3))
 (via (at 88 88.07) (size 0.8) (drill 0.4) (layers F.Cu B.Cu) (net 3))
 (via (at 98 103) (size 0.8) (drill 0.4) (layers F.Cu B.Cu) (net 3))
 (via (at 94 96) (size 0.8) (drill 0.4) (layers F.Cu B.Cu) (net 3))
 (via (at 115 105) (size 0.8) (drill 0.4) (layers F.Cu B.Cu) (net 3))
 (via (at 88 119) (size 0.8) (drill 0.4) (layers F.Cu B.Cu) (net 3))
 (via (at 87.07 89) (size 0.8) (drill 0.4) (layers F.Cu B.Cu) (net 3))
 (via (at 97 103) (size 0.8) (drill 0.4) (layers F.Cu B.Cu) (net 3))
 (via (at 95 95) (size 0.8) (drill 0.4) (layers F.Cu B.Cu) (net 3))
 (via (at 115 107) (size 0.8) (drill 0.4) (layers F.Cu B.Cu) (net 3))
 (via (at 87 119) (size 0.8) (drill 0.4) (layers F.Cu B.Cu) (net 3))
 (segment (start 42 32.982) (end 42 37.22) (width 0.8) (layer F.Cu) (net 2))
 (segment (start 122 51.25) (end 118.2 51.25) (width 0.8) (layer F.Cu) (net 2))
 (segment (start 43.562 31.42) (end 43.58 31.42) (width 0.8) (layer F.Cu) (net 2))
 (via (at 44 31) (size 0.8) (drill 0.4) (layers F.Cu B.Cu) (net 2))
 (segment (start 43.58 31.42) (end 44 31) (width 0.8) (layer F.Cu) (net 2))
 (segment (start 44 31) (end 45 32) (width 0.8) (layer B.Cu) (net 2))
 (segment (start 45 32) (end 44 33) (width 0.8) (layer B.Cu) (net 2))
 (segment (start 43 31.982) (end 43 32) (width 0.8) (layer F.Cu) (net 2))
 (segment (start 43 31.982) (end 42 32.982) (width 0.8) (layer F.Cu) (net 2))
 (segment (start 43.562 31.42) (end 43 31.982) (width 0.8) (layer F.Cu) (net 2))
 (via (at 44 33) (size 0.8) (drill 0.4) (layers F.Cu B.Cu) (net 2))
 (segment (start 43 32) (end 44 33) (width 0.8) (layer F.Cu) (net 2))
 (segment (start 45 32) (end 46 32) (width 0.8) (layer B.Cu) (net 2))
 (segment (start 46 32) (end 65 51) (width 0.8) (layer B.Cu) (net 2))
 (segment (start 65 51) (end 114 51) (width 0.8) (layer B.Cu) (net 2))
 (via (at 115 50) (size 0.8) (drill 0.4) (layers F.Cu B.Cu) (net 2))
 (segment (start 114 51) (end 115 50) (width 0.8) (layer B.Cu) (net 2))
 (segment (start 116.25 51.25) (end 118.2 51.25) (width 0.8) (layer F.Cu) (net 2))
 (segment (start 115 50) (end 116.25 51.25) (width 0.8) (layer F.Cu) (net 2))
 (via (at 115 52) (size 0.8) (drill 0.4) (layers F.Cu B.Cu) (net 2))
 (segment (start 114 51) (end 115 52) (width 0.8) (layer B.Cu) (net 2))
 (segment (start 115.75 51.25) (end 116.25 51.25) (width 0.8) (layer F.Cu) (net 2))
 (segment (start 115 52) (end 115.75 51.25) (width 0.8) (layer F.Cu) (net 2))
 (segment (start 44 81) (end 45 82) (width 0.8) (layer B.Cu) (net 2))
 (segment (start 115.75 101.25) (end 116.25 101.25) (width 0.8) (layer F.Cu) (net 2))
 (segment (start 43.562 81.42) (end 43.58 81.42) (width 0.8) (layer F.Cu) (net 2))
 (segment (start 45 82) (end 46 82) (width 0.8) (layer B.Cu) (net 2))
 (segment (start 115 100) (end 116.25 101.25) (width 0.8) (layer F.Cu) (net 2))
 (segment (start 45 82) (end 44 83) (width 0.8) (layer B.Cu) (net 2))
 (segment (start 43.562 81.42) (end 43 81.982) (width 0.8) (layer F.Cu) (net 2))
 (segment (start 122 101.25) (end 118.2 101.25) (width 0.8) (layer F.Cu) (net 2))
 (segment (start 43 81.982) (end 42 82.982) (width 0.8) (layer F.Cu) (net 2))
 (segment (start 114 101) (end 115 100) (width 0.8) (layer B.Cu) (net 2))
 (segment (start 116.25 101.25) (end 118.2 101.25) (width 0.8) (layer F.Cu) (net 2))
 (segment (start 115 102) (end 115.75 101.25) (width 0.8) (layer F.Cu) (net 2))
 (segment (start 114 101) (end 115 102) (width 0.8) (layer B.Cu) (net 2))
 (segment (start 65 101) (end 114 101) (width 0.8) (layer B.Cu) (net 2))
 (segment (start 43 82) (end 44 83) (width 0.8) (layer F.Cu) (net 2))
 (segment (start 46 82) (end 65 101) (width 0.8) (layer B.Cu) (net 2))
 (segment (start 43.58 81.42) (end 44 81) (width 0.8) (layer F.Cu) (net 2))
 (segment (start 43 81.982) (end 43 82) (width 0.8) (layer F.Cu) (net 2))
 (segment (start 42 82.982) (end 42 87.22) (width 0.8) (layer F.Cu) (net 2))
 (via (at 44 81) (size 0.8) (drill 0.4) (layers F.Cu B.Cu) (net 2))
 (via (at 115 100) (size 0.8) (drill 0.4) (layers F.Cu B.Cu) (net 2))
 (via (at 115 102) (size 0.8) (drill 0.4) (layers F.Cu B.Cu) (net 2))
 (via (at 44 83) (size 0.8) (drill 0.4) (layers F.Cu B.Cu) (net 2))
 (segment (start 90.81 75) (end 90.81 76.302002) (width 0.8) (layer F.Cu) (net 7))
 (segment (start 42 77.018) (end 42 72.78) (width 0.8) (layer F.Cu) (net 7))
 (segment (start 90.81 35) (end 90.81 68.81) (width 0.8) (layer F.Cu) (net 7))
 (segment (start 42 72.78) (end 43.78 72.78) (width 0.8) (layer F.Cu) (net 7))
 (via (at 44 72) (size 0.8) (drill 0.4) (layers F.Cu B.Cu) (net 7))
 (segment (start 43.78 72.78) (end 44 72.56) (width 0.8) (layer F.Cu) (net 7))
 (segment (start 44 72.56) (end 44 72) (width 0.8) (layer F.Cu) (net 7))
 (segment (start 44 72) (end 45 72) (width 0.8) (layer B.Cu) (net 7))
 (segment (start 45 72) (end 46 73) (width 0.8) (layer B.Cu) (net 7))
 (segment (start 46 73) (end 45 74) (width 0.8) (layer B.Cu) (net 7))
 (via (at 44 74) (size 0.8) (drill 0.4) (layers F.Cu B.Cu) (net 7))
 (segment (start 45 74) (end 44 74) (width 0.8) (layer B.Cu) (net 7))
 (segment (start 44 73) (end 43.78 72.78) (width 0.8) (layer F.Cu) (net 7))
 (segment (start 44 74) (end 44 73) (width 0.8) (layer F.Cu) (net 7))
 (segment (start 90.81 68.81) (end 90.81 69) (width 0.8) (layer F.Cu) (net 7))
 (via (at 90 71) (size 0.8) (drill 0.4) (layers F.Cu B.Cu) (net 7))
 (segment (start 88.414226 71) (end 90 71) (width 0.8) (layer B.Cu) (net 7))
 (segment (start 90 71) (end 90.81 71) (width 0.8) (layer F.Cu) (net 7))
 (segment (start 90.81 69) (end 90.81 71) (width 0.8) (layer F.Cu) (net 7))
 (segment (start 90.81 71) (end 90.81 75) (width 0.8) (layer F.Cu) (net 7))
 (via (at 89.000024 70) (size 0.8) (drill 0.4) (layers F.Cu B.Cu) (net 7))
 (segment (start 89.81 70) (end 89.565709 70) (width 0.8) (layer F.Cu) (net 7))
 (segment (start 88.565709 71) (end 89.000024 70.565685) (width 0.8) (layer B.Cu) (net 7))
 (segment (start 89.565709 70) (end 89.000024 70) (width 0.8) (layer F.Cu) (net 7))
 (segment (start 90.81 69) (end 89.81 70) (width 0.8) (layer F.Cu) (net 7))
 (segment (start 89.000024 70.565685) (end 89.000024 70) (width 0.8) (layer B.Cu) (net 7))
 (segment (start 88.414226 71) (end 88.565709 71) (width 0.8) (layer B.Cu) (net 7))
 (segment (start 45 124) (end 44 124) (width 0.8) (layer B.Cu) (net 7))
 (segment (start 90.81 119) (end 89.81 120) (width 0.8) (layer F.Cu) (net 7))
 (segment (start 42 122.78) (end 43.78 122.78) (width 0.8) (layer F.Cu) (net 7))
 (segment (start 44 122) (end 45 122) (width 0.8) (layer B.Cu) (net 7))
 (segment (start 87.514227 121.899999) (end 88.414226 121) (width 0.8) (layer B.Cu) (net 7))
 (segment (start 90.81 121) (end 90.81 125) (width 0.8) (layer F.Cu) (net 7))
 (segment (start 90.81 119) (end 90.81 121) (width 0.8) (layer F.Cu) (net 7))
 (segment (start 46 123) (end 45 124) (width 0.8) (layer B.Cu) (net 7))
 (segment (start 45 122) (end 46 123) (width 0.8) (layer B.Cu) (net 7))
 (segment (start 89.565709 120) (end 89.000024 120) (width 0.8) (layer F.Cu) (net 7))
 (segment (start 88.414226 121) (end 88.565709 121) (width 0.8) (layer B.Cu) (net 7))
 (segment (start 88.414226 121) (end 90 121) (width 0.8) (layer B.Cu) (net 7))
 (segment (start 43.78 122.78) (end 44 122.56) (width 0.8) (layer F.Cu) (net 7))
 (segment (start 88.565709 121) (end 89.000024 120.565685) (width 0.8) (layer B.Cu) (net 7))
 (segment (start 42 127.018) (end 42 122.78) (width 0.8) (layer F.Cu) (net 7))
 (segment (start 44 123) (end 43.78 122.78) (width 0.8) (layer F.Cu) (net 7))
 (segment (start 46 123) (end 47.100001 121.899999) (width 0.8) (layer B.Cu) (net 7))
 (segment (start 44 124) (end 44 123) (width 0.8) (layer F.Cu) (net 7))
 (segment (start 90.81 118.81) (end 90.81 119) (width 0.8) (layer F.Cu) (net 7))
 (segment (start 89.000024 120.565685) (end 89.000024 120) (width 0.8) (layer B.Cu) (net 7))
 (segment (start 90.81 125) (end 90.81 126.302002) (width 0.8) (layer F.Cu) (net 7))
 (segment (start 44 122.56) (end 44 122) (width 0.8) (layer F.Cu) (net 7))
 (segment (start 90.81 85) (end 90.81 118.81) (width 0.8) (layer F.Cu) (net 7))
 (segment (start 90 121) (end 90.81 121) (width 0.8) (layer F.Cu) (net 7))
 (segment (start 89.81 120) (end 89.565709 120) (width 0.8) (layer F.Cu) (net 7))
 (segment (start 47.100001 121.899999) (end 87.514227 121.899999) (width 0.8) (layer B.Cu) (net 7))
 (via (at 44 122) (size 0.8) (drill 0.4) (layers F.Cu B.Cu) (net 7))
 (via (at 44 124) (size 0.8) (drill 0.4) (layers F.Cu B.Cu) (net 7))
 (via (at 89.000024 120) (size 0.8) (drill 0.4) (layers F.Cu B.Cu) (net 7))
 (via (at 90 121) (size 0.8) (drill 0.4) (layers F.Cu B.Cu) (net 7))
 (segment (start 48 71) (end 88.414226 71) (width 0.8) (layer B.Cu) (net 7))
 (segment (start 46 73) (end 48 71) (width 0.8) (layer B.Cu) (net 7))
 (segment (start 93.35 75) (end 93.35 73.762) (width 0.25) (layer F.Cu) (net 1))
 (segment (start 102.112 75) (end 93.35 75) (width 0.25) (layer F.Cu) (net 1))
 (segment (start 114.492 62.62) (end 102.112 75) (width 0.25) (layer F.Cu) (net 1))
 (segment (start 125.984 62.62) (end 114.492 62.62) (width 0.25) (layer F.Cu) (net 1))
 (segment (start 125.984 50.484) (end 125.984 62.62) (width 0.25) (layer F.Cu) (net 1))
 (segment (start 122 48.75) (end 124.25 48.75) (width 0.25) (layer F.Cu) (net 1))
 (segment (start 124.25 48.75) (end 125.984 50.484) (width 0.25) (layer F.Cu) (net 1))
 (segment (start 93.35 36.238) (end 93.35 35) (width 0.25) (layer F.Cu) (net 1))
 (segment (start 105.862 48.75) (end 93.35 36.238) (width 0.25) (layer F.Cu) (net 1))
 (segment (start 122 48.75) (end 105.862 48.75) (width 0.25) (layer F.Cu) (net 1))
 (segment (start 93.35 86.238) (end 93.35 85) (width 0.25) (layer F.Cu) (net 1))
 (segment (start 125.984 112.62) (end 114.492 112.62) (width 0.25) (layer F.Cu) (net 1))
 (segment (start 102.112 125) (end 93.35 125) (width 0.25) (layer F.Cu) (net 1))
 (segment (start 122 98.75) (end 124.25 98.75) (width 0.25) (layer F.Cu) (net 1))
 (segment (start 124.25 98.75) (end 125.984 100.484) (width 0.25) (layer F.Cu) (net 1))
 (segment (start 125.984 100.484) (end 125.984 112.62) (width 0.25) (layer F.Cu) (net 1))
 (segment (start 93.35 125) (end 93.35 123.762) (width 0.25) (layer F.Cu) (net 1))
 (segment (start 114.492 112.62) (end 102.112 125) (width 0.25) (layer F.Cu) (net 1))
 (segment (start 105.862 98.75) (end 93.35 86.238) (width 0.25) (layer F.Cu) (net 1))
 (segment (start 122 98.75) (end 105.862 98.75) (width 0.25) (layer F.Cu) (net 1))
 (segment (start 47.562 72.78) (end 46 72.78) (width 0.8) (layer F.Cu) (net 6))
 (segment (start 49.086 71.256) (end 47.562 72.78) (width 0.8) (layer F.Cu) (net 6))
 (segment (start 80.684 71.256) (end 49.086 71.256) (width 0.8) (layer F.Cu) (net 6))
 (segment (start 80.65 75) (end 80.65 71.29) (width 0.8) (layer F.Cu) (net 6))
 (segment (start 80.65 71.29) (end 80.684 71.256) (width 0.8) (layer F.Cu) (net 6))
 (segment (start 80.65 71.29) (end 80.65 35) (width 0.8) (layer F.Cu) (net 6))
 (segment (start 49.086 121.256) (end 47.562 122.78) (width 0.8) (layer F.Cu) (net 6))
 (segment (start 80.684 121.256) (end 49.086 121.256) (width 0.8) (layer F.Cu) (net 6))
 (segment (start 47.562 122.78) (end 46 122.78) (width 0.8) (layer F.Cu) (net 6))
 (segment (start 80.65 125) (end 80.65 121.29) (width 0.8) (layer F.Cu) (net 6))
 (segment (start 80.65 121.29) (end 80.684 121.256) (width 0.8) (layer F.Cu) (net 6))
 (segment (start 80.65 121.29) (end 80.65 85) (width 0.8) (layer F.Cu) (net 6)))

